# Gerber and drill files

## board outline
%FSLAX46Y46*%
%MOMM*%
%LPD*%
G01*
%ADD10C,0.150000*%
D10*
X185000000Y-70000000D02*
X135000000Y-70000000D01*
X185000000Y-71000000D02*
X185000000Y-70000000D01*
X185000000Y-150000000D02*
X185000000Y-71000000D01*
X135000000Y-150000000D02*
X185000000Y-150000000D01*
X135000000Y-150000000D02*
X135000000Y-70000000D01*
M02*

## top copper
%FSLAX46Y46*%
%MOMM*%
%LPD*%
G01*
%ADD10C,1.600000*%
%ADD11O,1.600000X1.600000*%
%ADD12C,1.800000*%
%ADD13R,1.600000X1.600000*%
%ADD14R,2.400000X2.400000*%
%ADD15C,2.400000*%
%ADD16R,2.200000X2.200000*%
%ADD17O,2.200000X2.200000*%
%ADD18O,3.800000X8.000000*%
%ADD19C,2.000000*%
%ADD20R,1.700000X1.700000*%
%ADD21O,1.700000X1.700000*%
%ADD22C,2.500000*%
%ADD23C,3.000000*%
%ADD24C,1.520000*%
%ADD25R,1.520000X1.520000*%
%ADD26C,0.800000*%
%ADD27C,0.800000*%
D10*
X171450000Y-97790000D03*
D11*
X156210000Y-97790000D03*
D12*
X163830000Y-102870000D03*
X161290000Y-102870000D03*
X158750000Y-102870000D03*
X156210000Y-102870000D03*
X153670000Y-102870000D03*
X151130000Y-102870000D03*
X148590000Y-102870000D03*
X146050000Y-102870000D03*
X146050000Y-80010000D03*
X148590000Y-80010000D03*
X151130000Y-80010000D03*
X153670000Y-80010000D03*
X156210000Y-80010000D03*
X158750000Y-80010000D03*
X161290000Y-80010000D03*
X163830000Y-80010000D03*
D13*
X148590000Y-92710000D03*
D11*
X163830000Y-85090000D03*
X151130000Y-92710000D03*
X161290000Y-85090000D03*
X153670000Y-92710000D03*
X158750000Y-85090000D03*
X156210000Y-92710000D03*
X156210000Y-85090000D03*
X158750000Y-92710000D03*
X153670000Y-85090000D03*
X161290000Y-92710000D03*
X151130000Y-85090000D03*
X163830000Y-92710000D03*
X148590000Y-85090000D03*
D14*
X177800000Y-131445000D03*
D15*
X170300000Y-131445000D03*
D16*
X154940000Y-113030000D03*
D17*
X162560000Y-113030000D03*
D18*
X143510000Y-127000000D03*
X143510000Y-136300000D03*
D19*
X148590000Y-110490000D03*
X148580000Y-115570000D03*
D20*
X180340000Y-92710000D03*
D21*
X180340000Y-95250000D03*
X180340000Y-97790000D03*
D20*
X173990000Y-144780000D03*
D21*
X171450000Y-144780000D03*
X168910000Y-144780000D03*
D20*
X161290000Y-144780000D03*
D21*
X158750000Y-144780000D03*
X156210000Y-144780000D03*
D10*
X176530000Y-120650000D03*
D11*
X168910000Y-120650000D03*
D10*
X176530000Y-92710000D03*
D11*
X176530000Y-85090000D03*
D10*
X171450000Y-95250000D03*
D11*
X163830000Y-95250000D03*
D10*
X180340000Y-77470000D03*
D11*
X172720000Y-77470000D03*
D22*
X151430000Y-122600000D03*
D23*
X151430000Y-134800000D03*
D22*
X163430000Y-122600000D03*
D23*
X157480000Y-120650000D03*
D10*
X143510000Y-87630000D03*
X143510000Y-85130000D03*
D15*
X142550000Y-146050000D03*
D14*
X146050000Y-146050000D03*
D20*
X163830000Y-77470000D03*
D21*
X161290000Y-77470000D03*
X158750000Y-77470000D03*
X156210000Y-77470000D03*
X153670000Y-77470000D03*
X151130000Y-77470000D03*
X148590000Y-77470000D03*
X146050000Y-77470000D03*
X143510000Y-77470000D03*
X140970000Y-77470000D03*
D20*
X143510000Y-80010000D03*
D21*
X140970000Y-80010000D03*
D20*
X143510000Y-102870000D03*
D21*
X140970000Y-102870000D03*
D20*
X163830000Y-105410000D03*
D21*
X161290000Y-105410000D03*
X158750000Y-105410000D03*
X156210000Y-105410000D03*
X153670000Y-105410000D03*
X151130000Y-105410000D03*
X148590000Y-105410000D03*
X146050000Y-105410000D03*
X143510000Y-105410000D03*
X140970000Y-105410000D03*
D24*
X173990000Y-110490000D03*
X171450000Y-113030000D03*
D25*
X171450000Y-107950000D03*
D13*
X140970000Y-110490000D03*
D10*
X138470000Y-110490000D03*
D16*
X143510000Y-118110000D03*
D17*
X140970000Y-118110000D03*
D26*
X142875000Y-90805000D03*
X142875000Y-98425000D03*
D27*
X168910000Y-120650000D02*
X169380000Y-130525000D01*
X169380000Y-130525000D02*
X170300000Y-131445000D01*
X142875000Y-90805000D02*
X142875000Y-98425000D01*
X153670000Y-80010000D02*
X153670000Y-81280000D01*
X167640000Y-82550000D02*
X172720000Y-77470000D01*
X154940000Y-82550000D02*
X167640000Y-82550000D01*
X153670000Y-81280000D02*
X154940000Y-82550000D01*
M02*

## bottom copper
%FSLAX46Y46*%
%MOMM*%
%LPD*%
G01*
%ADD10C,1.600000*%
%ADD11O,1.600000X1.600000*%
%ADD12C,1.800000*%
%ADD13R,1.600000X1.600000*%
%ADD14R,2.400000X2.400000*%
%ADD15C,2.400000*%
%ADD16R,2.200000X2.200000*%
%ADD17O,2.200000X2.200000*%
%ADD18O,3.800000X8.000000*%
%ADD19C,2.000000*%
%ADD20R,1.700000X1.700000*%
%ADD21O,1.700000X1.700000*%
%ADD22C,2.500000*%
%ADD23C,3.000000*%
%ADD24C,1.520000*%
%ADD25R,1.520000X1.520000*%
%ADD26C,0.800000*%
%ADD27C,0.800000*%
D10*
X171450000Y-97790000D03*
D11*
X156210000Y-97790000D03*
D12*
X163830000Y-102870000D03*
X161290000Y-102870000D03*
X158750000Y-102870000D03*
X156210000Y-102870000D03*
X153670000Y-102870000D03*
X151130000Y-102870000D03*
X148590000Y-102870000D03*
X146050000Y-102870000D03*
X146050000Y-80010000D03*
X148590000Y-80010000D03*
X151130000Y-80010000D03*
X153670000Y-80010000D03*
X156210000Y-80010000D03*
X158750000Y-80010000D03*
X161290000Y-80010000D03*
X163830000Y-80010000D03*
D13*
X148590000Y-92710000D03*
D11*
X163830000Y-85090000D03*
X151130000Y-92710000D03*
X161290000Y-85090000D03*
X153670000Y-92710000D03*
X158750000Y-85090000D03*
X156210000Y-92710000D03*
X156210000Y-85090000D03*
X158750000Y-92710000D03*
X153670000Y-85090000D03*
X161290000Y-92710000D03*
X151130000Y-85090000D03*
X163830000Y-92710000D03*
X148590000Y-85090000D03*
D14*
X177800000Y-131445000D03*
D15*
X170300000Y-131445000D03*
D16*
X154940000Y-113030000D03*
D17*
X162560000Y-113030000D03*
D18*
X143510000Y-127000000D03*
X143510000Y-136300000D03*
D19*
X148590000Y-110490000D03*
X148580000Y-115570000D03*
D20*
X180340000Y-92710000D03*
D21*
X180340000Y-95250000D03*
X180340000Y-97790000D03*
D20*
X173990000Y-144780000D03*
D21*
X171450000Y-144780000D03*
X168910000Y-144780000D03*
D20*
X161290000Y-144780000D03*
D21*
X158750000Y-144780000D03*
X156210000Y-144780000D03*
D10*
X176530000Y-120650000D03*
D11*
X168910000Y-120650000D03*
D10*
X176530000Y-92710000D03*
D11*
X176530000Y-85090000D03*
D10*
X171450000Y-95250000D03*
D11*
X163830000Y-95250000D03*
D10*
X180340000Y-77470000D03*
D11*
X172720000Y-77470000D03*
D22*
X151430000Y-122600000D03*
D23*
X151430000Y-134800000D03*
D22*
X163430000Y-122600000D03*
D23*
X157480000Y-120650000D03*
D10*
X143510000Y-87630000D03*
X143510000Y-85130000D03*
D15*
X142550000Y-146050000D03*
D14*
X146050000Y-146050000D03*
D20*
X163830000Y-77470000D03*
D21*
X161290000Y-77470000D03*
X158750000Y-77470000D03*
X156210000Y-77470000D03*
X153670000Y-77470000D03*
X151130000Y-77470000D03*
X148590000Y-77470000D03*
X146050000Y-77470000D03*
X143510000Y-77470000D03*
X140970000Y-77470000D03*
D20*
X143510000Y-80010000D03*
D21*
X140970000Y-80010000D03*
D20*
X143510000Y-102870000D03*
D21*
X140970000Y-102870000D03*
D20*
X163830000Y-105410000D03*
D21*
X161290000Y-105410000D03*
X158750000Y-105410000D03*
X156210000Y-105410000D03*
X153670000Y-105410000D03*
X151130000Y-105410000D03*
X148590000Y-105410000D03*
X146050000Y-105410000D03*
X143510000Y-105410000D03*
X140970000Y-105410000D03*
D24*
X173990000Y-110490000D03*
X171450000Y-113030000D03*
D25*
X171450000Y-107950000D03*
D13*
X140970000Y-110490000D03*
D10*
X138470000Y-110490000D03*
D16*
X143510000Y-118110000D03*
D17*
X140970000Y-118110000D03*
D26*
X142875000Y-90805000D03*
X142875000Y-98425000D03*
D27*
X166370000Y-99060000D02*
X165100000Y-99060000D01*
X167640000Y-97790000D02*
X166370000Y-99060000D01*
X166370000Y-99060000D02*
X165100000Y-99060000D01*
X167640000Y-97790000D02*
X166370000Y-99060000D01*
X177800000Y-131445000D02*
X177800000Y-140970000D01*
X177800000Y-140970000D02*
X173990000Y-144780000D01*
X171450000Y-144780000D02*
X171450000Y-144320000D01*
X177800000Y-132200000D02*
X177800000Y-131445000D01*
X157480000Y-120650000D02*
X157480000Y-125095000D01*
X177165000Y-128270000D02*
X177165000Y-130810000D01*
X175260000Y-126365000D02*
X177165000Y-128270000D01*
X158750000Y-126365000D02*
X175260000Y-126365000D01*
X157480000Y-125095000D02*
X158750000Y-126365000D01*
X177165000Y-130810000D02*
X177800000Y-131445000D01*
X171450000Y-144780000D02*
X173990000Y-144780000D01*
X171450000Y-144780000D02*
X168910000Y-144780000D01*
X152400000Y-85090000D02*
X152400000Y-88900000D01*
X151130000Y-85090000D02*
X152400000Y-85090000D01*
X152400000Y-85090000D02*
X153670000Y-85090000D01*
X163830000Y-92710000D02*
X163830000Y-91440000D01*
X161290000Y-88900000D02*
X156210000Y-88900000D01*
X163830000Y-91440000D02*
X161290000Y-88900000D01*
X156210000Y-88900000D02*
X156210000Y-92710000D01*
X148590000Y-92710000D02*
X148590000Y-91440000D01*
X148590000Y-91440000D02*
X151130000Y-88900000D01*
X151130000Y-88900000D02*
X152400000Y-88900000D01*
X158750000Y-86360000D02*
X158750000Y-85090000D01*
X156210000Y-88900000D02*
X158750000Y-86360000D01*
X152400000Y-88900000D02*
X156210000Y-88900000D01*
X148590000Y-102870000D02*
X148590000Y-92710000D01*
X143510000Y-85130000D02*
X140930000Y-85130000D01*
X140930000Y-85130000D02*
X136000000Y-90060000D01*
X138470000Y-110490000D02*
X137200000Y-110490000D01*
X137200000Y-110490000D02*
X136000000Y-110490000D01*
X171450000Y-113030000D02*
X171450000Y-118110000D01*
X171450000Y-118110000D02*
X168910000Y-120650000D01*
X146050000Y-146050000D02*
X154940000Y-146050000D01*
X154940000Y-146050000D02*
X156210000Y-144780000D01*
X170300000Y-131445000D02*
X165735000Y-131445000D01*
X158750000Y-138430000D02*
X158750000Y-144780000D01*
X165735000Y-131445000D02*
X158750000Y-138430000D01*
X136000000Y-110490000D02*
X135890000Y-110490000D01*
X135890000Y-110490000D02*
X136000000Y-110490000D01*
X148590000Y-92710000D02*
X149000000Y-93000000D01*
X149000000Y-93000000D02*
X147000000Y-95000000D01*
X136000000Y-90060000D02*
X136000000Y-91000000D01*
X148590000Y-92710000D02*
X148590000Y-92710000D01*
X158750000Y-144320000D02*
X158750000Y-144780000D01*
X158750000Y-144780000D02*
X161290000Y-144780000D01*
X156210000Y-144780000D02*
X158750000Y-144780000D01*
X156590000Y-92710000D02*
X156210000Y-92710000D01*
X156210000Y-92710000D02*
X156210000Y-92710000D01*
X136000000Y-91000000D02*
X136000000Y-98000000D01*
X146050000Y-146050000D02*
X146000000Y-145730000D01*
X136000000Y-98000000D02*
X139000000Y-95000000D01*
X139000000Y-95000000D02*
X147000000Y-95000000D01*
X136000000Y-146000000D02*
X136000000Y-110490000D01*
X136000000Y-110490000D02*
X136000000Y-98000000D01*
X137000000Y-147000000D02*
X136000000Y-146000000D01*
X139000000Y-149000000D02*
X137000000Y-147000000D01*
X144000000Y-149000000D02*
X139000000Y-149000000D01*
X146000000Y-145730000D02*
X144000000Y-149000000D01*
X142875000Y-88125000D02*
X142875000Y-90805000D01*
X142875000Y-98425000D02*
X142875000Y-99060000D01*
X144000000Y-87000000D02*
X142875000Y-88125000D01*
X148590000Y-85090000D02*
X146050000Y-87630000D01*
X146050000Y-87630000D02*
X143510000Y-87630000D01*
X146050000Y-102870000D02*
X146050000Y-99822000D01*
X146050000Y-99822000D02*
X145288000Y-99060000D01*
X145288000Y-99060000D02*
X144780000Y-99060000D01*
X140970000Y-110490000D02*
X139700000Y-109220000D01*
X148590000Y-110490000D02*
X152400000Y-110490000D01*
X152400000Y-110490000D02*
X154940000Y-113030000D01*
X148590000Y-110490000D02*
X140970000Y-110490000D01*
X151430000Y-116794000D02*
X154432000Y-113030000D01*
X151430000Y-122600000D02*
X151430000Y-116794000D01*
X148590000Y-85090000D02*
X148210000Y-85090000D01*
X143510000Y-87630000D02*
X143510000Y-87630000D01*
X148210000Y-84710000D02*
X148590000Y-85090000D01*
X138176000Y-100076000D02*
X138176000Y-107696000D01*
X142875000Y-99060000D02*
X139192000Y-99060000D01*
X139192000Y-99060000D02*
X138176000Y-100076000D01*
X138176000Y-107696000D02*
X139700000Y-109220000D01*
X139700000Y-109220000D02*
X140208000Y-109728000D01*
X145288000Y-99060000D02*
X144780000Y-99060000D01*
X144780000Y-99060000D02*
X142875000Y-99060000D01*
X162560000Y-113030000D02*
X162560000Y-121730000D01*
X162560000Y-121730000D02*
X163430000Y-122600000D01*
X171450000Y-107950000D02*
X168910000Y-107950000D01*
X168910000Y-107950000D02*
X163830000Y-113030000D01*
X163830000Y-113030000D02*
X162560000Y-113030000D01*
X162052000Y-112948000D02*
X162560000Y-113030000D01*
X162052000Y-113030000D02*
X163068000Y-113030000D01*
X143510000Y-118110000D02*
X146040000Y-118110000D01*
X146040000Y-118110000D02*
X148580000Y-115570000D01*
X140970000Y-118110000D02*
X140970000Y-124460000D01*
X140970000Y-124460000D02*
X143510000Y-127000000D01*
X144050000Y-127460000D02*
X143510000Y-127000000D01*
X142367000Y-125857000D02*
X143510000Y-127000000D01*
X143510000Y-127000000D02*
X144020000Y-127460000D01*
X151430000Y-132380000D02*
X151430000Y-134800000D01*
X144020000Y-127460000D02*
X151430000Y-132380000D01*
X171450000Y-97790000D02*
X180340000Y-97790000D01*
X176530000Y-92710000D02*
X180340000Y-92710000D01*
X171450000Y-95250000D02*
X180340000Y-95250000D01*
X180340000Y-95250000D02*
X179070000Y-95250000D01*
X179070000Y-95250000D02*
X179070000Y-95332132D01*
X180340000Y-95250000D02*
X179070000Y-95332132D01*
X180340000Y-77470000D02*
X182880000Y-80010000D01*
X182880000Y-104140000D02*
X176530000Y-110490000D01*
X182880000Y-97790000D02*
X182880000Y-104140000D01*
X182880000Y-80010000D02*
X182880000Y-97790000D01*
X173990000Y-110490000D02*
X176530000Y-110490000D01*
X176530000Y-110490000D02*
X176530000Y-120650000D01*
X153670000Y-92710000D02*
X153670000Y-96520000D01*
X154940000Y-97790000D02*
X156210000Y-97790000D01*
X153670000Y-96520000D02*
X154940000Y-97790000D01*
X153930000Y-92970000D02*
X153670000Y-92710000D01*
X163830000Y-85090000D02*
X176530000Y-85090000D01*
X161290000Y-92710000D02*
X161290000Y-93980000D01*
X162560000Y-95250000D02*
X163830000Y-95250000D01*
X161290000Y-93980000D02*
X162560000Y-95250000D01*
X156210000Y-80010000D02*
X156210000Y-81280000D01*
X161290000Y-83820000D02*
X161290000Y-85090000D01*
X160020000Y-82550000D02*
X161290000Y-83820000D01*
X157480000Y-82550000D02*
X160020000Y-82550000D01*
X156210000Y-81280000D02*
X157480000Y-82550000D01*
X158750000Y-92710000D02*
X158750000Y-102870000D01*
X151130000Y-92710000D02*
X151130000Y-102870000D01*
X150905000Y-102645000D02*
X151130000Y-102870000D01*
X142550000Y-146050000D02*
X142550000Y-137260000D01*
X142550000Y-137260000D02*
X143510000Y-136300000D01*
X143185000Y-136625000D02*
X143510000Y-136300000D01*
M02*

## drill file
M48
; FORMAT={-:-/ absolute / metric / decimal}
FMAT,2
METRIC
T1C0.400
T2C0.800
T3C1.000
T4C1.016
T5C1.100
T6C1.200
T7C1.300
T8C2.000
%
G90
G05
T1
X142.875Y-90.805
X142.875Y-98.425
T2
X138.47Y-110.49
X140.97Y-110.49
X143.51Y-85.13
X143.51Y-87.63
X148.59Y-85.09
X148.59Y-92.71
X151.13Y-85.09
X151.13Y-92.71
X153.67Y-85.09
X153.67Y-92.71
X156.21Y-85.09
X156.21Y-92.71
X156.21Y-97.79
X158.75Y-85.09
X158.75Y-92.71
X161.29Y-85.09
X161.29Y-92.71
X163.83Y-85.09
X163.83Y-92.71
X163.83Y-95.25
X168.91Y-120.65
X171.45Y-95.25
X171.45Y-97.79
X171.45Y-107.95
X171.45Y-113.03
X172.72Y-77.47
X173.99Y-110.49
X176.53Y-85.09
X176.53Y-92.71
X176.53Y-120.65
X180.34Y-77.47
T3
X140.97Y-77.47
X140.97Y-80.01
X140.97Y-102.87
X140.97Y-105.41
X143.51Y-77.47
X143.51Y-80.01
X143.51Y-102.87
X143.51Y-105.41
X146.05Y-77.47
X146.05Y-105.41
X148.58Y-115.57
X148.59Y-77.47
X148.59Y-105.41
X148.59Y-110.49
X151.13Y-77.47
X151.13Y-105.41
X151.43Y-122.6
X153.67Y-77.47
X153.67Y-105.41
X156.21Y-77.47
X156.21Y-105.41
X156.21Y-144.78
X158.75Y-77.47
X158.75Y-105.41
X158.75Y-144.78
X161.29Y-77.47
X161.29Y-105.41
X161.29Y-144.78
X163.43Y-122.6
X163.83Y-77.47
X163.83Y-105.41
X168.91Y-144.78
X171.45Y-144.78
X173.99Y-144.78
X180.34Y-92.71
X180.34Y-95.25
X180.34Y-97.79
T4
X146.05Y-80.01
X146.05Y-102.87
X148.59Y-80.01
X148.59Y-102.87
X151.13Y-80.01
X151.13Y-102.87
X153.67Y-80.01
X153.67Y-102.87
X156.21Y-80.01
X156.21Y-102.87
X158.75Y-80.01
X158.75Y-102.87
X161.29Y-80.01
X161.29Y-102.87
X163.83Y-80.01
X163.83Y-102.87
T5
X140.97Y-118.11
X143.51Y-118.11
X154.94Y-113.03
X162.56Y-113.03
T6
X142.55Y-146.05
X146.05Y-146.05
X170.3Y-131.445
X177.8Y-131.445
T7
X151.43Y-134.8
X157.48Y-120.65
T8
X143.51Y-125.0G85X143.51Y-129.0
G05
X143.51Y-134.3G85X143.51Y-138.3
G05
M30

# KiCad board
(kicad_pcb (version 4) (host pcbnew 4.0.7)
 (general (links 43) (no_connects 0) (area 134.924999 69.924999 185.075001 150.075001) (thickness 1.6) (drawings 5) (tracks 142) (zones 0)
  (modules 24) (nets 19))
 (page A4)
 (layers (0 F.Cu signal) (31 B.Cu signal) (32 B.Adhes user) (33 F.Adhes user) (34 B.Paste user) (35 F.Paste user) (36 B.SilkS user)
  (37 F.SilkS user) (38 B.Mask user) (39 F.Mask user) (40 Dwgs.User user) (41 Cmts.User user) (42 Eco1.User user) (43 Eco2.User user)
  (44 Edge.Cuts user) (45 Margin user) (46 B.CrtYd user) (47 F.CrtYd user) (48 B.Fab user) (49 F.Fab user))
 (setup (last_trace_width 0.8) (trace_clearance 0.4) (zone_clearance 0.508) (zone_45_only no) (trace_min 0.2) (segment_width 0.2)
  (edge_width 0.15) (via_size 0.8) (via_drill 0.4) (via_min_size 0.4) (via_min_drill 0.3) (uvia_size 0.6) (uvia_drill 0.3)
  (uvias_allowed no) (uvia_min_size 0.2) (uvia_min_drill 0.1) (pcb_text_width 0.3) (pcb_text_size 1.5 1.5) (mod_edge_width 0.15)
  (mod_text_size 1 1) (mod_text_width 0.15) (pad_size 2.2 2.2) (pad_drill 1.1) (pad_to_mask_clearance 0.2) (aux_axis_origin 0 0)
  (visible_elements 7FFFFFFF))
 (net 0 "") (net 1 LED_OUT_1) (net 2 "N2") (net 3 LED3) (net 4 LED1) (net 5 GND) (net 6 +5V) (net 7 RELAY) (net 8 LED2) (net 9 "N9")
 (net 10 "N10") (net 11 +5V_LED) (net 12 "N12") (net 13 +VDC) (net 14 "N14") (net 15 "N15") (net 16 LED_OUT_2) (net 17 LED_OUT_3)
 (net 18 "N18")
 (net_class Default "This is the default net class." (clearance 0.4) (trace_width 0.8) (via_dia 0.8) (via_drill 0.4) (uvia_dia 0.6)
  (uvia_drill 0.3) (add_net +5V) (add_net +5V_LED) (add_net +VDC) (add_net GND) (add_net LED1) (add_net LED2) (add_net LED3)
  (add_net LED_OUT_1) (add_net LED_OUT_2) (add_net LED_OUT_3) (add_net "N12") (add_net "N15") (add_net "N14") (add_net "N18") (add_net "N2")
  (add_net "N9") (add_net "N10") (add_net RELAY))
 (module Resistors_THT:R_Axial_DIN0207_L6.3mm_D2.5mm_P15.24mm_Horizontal (layer F.Cu) (at 171.45 97.79 180)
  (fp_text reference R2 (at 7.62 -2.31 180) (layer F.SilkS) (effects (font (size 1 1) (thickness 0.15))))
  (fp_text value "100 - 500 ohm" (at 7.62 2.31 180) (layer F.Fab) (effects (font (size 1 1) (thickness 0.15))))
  (pad 1 thru_hole circle (at 0 0 180) (size 1.6 1.6) (drill 0.8) (layers *.Cu *.Mask) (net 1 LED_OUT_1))
  (pad 2 thru_hole oval (at 15.24 0 180) (size 1.6 1.6) (drill 0.8) (layers *.Cu *.Mask) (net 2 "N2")))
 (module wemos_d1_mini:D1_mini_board (layer B.Cu) (at 153.67 91.44 90)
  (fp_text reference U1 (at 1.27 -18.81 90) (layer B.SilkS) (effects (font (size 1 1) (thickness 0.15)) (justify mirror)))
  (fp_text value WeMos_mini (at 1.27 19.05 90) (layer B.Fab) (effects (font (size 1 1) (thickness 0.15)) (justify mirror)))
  (pad 8 thru_hole circle (at -11.43 10.16 90) (size 1.8 1.8) (drill 1.016) (layers *.Cu *.Mask B.SilkS))
  (pad 7 thru_hole circle (at -11.43 7.62 90) (size 1.8 1.8) (drill 1.016) (layers *.Cu *.Mask B.SilkS))
  (pad 6 thru_hole circle (at -11.43 5.08 90) (size 1.8 1.8) (drill 1.016) (layers *.Cu *.Mask B.SilkS) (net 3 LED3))
  (pad 5 thru_hole circle (at -11.43 2.54 90) (size 1.8 1.8) (drill 1.016) (layers *.Cu *.Mask B.SilkS))
  (pad 4 thru_hole circle (at -11.43 0 90) (size 1.8 1.8) (drill 1.016) (layers *.Cu *.Mask B.SilkS))
  (pad 3 thru_hole circle (at -11.43 -2.54 90) (size 1.8 1.8) (drill 1.016) (layers *.Cu *.Mask B.SilkS) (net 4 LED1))
  (pad 2 thru_hole circle (at -11.43 -5.08 90) (size 1.8 1.8) (drill 1.016) (layers *.Cu *.Mask B.SilkS) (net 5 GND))
  (pad 1 thru_hole circle (at -11.43 -7.62 90) (size 1.8 1.8) (drill 1.016) (layers *.Cu *.Mask B.SilkS) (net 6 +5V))
  (pad 16 thru_hole circle (at 11.43 -7.62 90) (size 1.8 1.8) (drill 1.016) (layers *.Cu *.Mask B.SilkS))
  (pad 15 thru_hole circle (at 11.43 -5.08 90) (size 1.8 1.8) (drill 1.016) (layers *.Cu *.Mask B.SilkS))
  (pad 14 thru_hole circle (at 11.43 -2.54 90) (size 1.8 1.8) (drill 1.016) (layers *.Cu *.Mask B.SilkS))
  (pad 13 thru_hole circle (at 11.43 0 90) (size 1.8 1.8) (drill 1.016) (layers *.Cu *.Mask B.SilkS) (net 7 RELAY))
  (pad 12 thru_hole circle (at 11.43 2.54 90) (size 1.8 1.8) (drill 1.016) (layers *.Cu *.Mask B.SilkS) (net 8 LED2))
  (pad 11 thru_hole circle (at 11.43 5.08 90) (size 1.8 1.8) (drill 1.016) (layers *.Cu *.Mask B.SilkS))
  (pad 10 thru_hole circle (at 11.43 7.62 90) (size 1.8 1.8) (drill 1.016) (layers *.Cu *.Mask B.SilkS))
  (pad 9 thru_hole circle (at 11.43 10.16 90) (size 1.8 1.8) (drill 1.016) (layers *.Cu *.Mask B.SilkS)))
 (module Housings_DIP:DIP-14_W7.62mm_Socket (layer F.Cu) (at 148.59 92.71 90)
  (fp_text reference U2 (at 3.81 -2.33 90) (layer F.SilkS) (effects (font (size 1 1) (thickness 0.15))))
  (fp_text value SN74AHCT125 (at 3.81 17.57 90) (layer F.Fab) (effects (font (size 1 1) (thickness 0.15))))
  (pad 1 thru_hole rect (at 0 0 90) (size 1.6 1.6) (drill 0.8) (layers *.Cu *.Mask) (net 5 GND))
  (pad 8 thru_hole oval (at 7.62 15.24 90) (size 1.6 1.6) (drill 0.8) (layers *.Cu *.Mask) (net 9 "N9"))
  (pad 2 thru_hole oval (at 0 2.54 90) (size 1.6 1.6) (drill 0.8) (layers *.Cu *.Mask) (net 4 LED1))
  (pad 9 thru_hole oval (at 7.62 12.7 90) (size 1.6 1.6) (drill 0.8) (layers *.Cu *.Mask) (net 8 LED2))
  (pad 3 thru_hole oval (at 0 5.08 90) (size 1.6 1.6) (drill 0.8) (layers *.Cu *.Mask) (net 2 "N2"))
  (pad 10 thru_hole oval (at 7.62 10.16 90) (size 1.6 1.6) (drill 0.8) (layers *.Cu *.Mask) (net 5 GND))
  (pad 4 thru_hole oval (at 0 7.62 90) (size 1.6 1.6) (drill 0.8) (layers *.Cu *.Mask) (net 5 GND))
  (pad 11 thru_hole oval (at 7.62 7.62 90) (size 1.6 1.6) (drill 0.8) (layers *.Cu *.Mask))
  (pad 5 thru_hole oval (at 0 10.16 90) (size 1.6 1.6) (drill 0.8) (layers *.Cu *.Mask) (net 3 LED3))
  (pad 12 thru_hole oval (at 7.62 5.08 90) (size 1.6 1.6) (drill 0.8) (layers *.Cu *.Mask) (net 5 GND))
  (pad 6 thru_hole oval (at 0 12.7 90) (size 1.6 1.6) (drill 0.8) (layers *.Cu *.Mask) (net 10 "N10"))
  (pad 13 thru_hole oval (at 7.62 2.54 90) (size 1.6 1.6) (drill 0.8) (layers *.Cu *.Mask) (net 5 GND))
  (pad 7 thru_hole oval (at 0 15.24 90) (size 1.6 1.6) (drill 0.8) (layers *.Cu *.Mask) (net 5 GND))
  (pad 14 thru_hole oval (at 7.62 0 90) (size 1.6 1.6) (drill 0.8) (layers *.Cu *.Mask) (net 6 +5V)))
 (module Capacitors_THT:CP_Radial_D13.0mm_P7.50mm (layer F.Cu) (at 177.8 131.445 180)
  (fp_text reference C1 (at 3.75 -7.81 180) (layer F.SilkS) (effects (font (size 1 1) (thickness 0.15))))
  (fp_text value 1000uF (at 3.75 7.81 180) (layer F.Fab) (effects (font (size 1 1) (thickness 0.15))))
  (pad 1 thru_hole rect (at 0 0 180) (size 2.4 2.4) (drill 1.2) (layers *.Cu *.Mask) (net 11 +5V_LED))
  (pad 2 thru_hole circle (at 7.5 0 180) (size 2.4 2.4) (drill 1.2) (layers *.Cu *.Mask) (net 5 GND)))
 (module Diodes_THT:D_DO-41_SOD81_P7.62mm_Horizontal (layer F.Cu) (at 154.94 113.03)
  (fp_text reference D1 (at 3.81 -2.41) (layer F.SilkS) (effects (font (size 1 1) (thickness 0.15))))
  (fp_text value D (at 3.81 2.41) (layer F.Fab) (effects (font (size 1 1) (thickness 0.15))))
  (pad 1 thru_hole rect (at 0 0) (size 2.2 2.2) (drill 1.1) (layers *.Cu *.Mask) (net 6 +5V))
  (pad 2 thru_hole oval (at 7.62 0) (size 2.2 2.2) (drill 1.1) (layers *.Cu *.Mask) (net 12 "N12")))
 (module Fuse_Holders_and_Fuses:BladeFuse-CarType (layer F.Cu) (at 143.51 127 270)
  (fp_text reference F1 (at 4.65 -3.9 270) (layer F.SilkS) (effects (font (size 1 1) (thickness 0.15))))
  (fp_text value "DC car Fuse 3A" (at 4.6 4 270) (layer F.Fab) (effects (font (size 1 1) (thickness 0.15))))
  (pad 1 thru_hole oval (at 0 0 270) (size 8 3.8) (drill oval 6 2) (layers *.Cu *.Mask) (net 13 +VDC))
  (pad 2 thru_hole oval (at 9.3 0 270) (size 8 3.8) (drill oval 6 2) (layers *.Cu *.Mask) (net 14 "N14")))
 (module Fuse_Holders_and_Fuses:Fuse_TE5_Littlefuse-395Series (layer F.Cu) (at 148.59 110.49 270)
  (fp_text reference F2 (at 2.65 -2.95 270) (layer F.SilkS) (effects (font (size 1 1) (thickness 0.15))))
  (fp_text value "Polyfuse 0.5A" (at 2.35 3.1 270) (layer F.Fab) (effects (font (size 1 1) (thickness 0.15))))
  (pad 1 thru_hole circle (at 0 0 270) (size 2 2) (drill 1) (layers *.Cu *.Mask) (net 6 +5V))
  (pad 2 thru_hole circle (at 5.08 0.01 270) (size 2 2) (drill 1) (layers *.Cu *.Mask) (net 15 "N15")))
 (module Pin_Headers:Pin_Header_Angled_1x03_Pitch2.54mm (layer F.Cu) (at 180.34 92.71)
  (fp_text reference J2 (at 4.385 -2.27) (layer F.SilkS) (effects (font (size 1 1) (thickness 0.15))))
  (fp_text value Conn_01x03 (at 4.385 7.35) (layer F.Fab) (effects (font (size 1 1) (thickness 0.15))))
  (pad 1 thru_hole rect (at 0 0) (size 1.7 1.7) (drill 1) (layers *.Cu *.Mask) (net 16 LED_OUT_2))
  (pad 2 thru_hole oval (at 0 2.54) (size 1.7 1.7) (drill 1) (layers *.Cu *.Mask) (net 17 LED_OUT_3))
  (pad 3 thru_hole oval (at 0 5.08) (size 1.7 1.7) (drill 1) (layers *.Cu *.Mask) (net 1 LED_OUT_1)))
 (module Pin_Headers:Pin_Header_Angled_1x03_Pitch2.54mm (layer F.Cu) (at 173.99 144.78 270)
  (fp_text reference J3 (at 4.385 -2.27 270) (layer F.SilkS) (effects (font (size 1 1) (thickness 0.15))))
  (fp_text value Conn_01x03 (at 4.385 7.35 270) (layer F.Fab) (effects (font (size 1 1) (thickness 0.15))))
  (pad 1 thru_hole rect (at 0 0 270) (size 1.7 1.7) (drill 1) (layers *.Cu *.Mask) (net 11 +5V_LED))
  (pad 2 thru_hole oval (at 0 2.54 270) (size 1.7 1.7) (drill 1) (layers *.Cu *.Mask) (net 11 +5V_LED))
  (pad 3 thru_hole oval (at 0 5.08 270) (size 1.7 1.7) (drill 1) (layers *.Cu *.Mask) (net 11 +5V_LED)))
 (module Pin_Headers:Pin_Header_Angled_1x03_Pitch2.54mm (layer F.Cu) (at 161.29 144.78 270)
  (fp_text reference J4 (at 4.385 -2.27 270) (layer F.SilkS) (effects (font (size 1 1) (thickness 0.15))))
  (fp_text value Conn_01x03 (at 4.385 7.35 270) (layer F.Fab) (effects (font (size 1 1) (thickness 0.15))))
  (pad 1 thru_hole rect (at 0 0 270) (size 1.7 1.7) (drill 1) (layers *.Cu *.Mask) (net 5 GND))
  (pad 2 thru_hole oval (at 0 2.54 270) (size 1.7 1.7) (drill 1) (layers *.Cu *.Mask) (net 5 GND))
  (pad 3 thru_hole oval (at 0 5.08 270) (size 1.7 1.7) (drill 1) (layers *.Cu *.Mask) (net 5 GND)))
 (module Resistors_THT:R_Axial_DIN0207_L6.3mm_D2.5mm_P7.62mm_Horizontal (layer F.Cu) (at 176.53 120.65 180)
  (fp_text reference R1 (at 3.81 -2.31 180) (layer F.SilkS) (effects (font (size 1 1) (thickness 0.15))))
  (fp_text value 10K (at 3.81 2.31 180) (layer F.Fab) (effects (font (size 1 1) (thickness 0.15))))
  (pad 1 thru_hole circle (at 0 0 180) (size 1.6 1.6) (drill 0.8) (layers *.Cu *.Mask) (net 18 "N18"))
  (pad 2 thru_hole oval (at 7.62 0 180) (size 1.6 1.6) (drill 0.8) (layers *.Cu *.Mask) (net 5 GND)))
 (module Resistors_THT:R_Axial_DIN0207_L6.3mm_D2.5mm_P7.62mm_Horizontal (layer F.Cu) (at 176.53 92.71 90)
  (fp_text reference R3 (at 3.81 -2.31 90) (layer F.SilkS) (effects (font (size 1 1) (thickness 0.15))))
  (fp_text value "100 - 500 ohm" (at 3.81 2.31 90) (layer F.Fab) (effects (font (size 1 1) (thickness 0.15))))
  (pad 1 thru_hole circle (at 0 0 90) (size 1.6 1.6) (drill 0.8) (layers *.Cu *.Mask) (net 16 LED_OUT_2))
  (pad 2 thru_hole oval (at 7.62 0 90) (size 1.6 1.6) (drill 0.8) (layers *.Cu *.Mask) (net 9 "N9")))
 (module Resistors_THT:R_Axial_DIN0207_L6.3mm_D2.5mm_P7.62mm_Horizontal (layer F.Cu) (at 171.45 95.25 180)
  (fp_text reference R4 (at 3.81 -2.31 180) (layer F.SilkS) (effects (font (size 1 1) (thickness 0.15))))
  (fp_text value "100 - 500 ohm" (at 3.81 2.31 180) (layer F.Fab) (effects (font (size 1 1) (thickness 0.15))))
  (pad 1 thru_hole circle (at 0 0 180) (size 1.6 1.6) (drill 0.8) (layers *.Cu *.Mask) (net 17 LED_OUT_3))
  (pad 2 thru_hole oval (at 7.62 0 180) (size 1.6 1.6) (drill 0.8) (layers *.Cu *.Mask) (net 10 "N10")))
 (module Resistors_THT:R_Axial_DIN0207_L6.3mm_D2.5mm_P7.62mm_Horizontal (layer F.Cu) (at 180.34 77.47 180)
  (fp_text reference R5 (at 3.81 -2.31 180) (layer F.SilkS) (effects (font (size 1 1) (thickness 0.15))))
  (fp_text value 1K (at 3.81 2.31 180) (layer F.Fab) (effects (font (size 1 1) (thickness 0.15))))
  (pad 1 thru_hole circle (at 0 0 180) (size 1.6 1.6) (drill 0.8) (layers *.Cu *.Mask) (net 18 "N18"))
  (pad 2 thru_hole oval (at 7.62 0 180) (size 1.6 1.6) (drill 0.8) (layers *.Cu *.Mask) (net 7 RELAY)))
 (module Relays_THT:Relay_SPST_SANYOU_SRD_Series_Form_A (layer F.Cu) (at 157.48 120.65 270)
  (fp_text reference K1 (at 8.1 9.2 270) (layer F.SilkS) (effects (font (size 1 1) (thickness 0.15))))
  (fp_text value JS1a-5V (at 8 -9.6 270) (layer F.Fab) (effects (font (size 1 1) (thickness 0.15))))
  (pad 5 thru_hole circle (at 1.95 6.05) (size 2.5 2.5) (drill 1) (layers *.Cu *.Mask) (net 6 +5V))
  (pad 4 thru_hole circle (at 14.15 6.05) (size 3 3) (drill 1.3) (layers *.Cu *.Mask) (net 13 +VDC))
  (pad 2 thru_hole circle (at 1.95 -5.95) (size 2.5 2.5) (drill 1) (layers *.Cu *.Mask) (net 12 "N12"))
  (pad 1 thru_hole circle (at 0 0) (size 3 3) (drill 1.3) (layers *.Cu *.Mask) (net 11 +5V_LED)))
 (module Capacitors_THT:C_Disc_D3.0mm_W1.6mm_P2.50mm (layer F.Cu) (at 143.51 87.63 90)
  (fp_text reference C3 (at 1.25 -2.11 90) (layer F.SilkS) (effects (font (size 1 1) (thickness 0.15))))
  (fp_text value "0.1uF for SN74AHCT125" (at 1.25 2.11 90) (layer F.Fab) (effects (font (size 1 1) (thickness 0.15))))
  (pad 1 thru_hole circle (at 0 0 90) (size 1.6 1.6) (drill 0.8) (layers *.Cu *.Mask) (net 6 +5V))
  (pad 2 thru_hole circle (at 2.5 0 90) (size 1.6 1.6) (drill 0.8) (layers *.Cu *.Mask) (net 5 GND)))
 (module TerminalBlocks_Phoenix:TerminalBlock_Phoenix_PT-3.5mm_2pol (layer F.Cu) (at 146.05 146.05 180)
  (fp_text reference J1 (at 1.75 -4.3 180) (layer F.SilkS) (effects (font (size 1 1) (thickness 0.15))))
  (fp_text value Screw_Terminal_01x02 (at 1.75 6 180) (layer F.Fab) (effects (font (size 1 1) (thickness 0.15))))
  (pad 2 thru_hole circle (at 3.5 0 180) (size 2.4 2.4) (drill 1.2) (layers *.Cu *.Mask) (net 14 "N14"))
  (pad 1 thru_hole rect (at 0 0 180) (size 2.4 2.4) (drill 1.2) (layers *.Cu *.Mask) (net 5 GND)))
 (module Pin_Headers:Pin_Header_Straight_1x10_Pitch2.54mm (layer F.Cu) (at 163.83 77.47 270)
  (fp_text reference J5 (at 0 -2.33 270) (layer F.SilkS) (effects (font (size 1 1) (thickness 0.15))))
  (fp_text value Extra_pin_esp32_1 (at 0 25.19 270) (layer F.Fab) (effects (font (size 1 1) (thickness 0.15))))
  (pad 1 thru_hole rect (at 0 0 270) (size 1.7 1.7) (drill 1) (layers *.Cu *.Mask))
  (pad 2 thru_hole oval (at 0 2.54 270) (size 1.7 1.7) (drill 1) (layers *.Cu *.Mask))
  (pad 3 thru_hole oval (at 0 5.08 270) (size 1.7 1.7) (drill 1) (layers *.Cu *.Mask))
  (pad 4 thru_hole oval (at 0 7.62 270) (size 1.7 1.7) (drill 1) (layers *.Cu *.Mask))
  (pad 5 thru_hole oval (at 0 10.16 270) (size 1.7 1.7) (drill 1) (layers *.Cu *.Mask))
  (pad 6 thru_hole oval (at 0 12.7 270) (size 1.7 1.7) (drill 1) (layers *.Cu *.Mask))
  (pad 7 thru_hole oval (at 0 15.24 270) (size 1.7 1.7) (drill 1) (layers *.Cu *.Mask))
  (pad 8 thru_hole oval (at 0 17.78 270) (size 1.7 1.7) (drill 1) (layers *.Cu *.Mask))
  (pad 9 thru_hole oval (at 0 20.32 270) (size 1.7 1.7) (drill 1) (layers *.Cu *.Mask))
  (pad 10 thru_hole oval (at 0 22.86 270) (size 1.7 1.7) (drill 1) (layers *.Cu *.Mask)))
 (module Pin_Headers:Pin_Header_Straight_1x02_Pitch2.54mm (layer F.Cu) (at 143.51 80.01 270)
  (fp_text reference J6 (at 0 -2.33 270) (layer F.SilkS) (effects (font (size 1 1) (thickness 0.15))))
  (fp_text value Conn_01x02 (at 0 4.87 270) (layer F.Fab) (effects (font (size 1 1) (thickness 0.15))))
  (pad 1 thru_hole rect (at 0 0 270) (size 1.7 1.7) (drill 1) (layers *.Cu *.Mask))
  (pad 2 thru_hole oval (at 0 2.54 270) (size 1.7 1.7) (drill 1) (layers *.Cu *.Mask)))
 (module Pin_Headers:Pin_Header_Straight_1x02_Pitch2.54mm (layer F.Cu) (at 143.51 102.87 270)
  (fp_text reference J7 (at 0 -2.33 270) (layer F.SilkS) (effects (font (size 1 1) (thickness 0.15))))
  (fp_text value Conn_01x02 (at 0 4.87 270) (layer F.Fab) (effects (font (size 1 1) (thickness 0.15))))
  (pad 1 thru_hole rect (at 0 0 270) (size 1.7 1.7) (drill 1) (layers *.Cu *.Mask))
  (pad 2 thru_hole oval (at 0 2.54 270) (size 1.7 1.7) (drill 1) (layers *.Cu *.Mask)))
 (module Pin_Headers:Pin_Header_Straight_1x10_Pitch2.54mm (layer F.Cu) (at 163.83 105.41 270)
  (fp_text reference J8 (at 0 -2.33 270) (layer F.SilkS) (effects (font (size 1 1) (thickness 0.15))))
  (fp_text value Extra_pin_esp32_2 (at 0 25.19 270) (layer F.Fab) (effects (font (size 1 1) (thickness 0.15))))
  (pad 1 thru_hole rect (at 0 0 270) (size 1.7 1.7) (drill 1) (layers *.Cu *.Mask))
  (pad 2 thru_hole oval (at 0 2.54 270) (size 1.7 1.7) (drill 1) (layers *.Cu *.Mask))
  (pad 3 thru_hole oval (at 0 5.08 270) (size 1.7 1.7) (drill 1) (layers *.Cu *.Mask))
  (pad 4 thru_hole oval (at 0 7.62 270) (size 1.7 1.7) (drill 1) (layers *.Cu *.Mask))
  (pad 5 thru_hole oval (at 0 10.16 270) (size 1.7 1.7) (drill 1) (layers *.Cu *.Mask))
  (pad 6 thru_hole oval (at 0 12.7 270) (size 1.7 1.7) (drill 1) (layers *.Cu *.Mask))
  (pad 7 thru_hole oval (at 0 15.24 270) (size 1.7 1.7) (drill 1) (layers *.Cu *.Mask))
  (pad 8 thru_hole oval (at 0 17.78 270) (size 1.7 1.7) (drill 1) (layers *.Cu *.Mask))
  (pad 9 thru_hole oval (at 0 20.32 270) (size 1.7 1.7) (drill 1) (layers *.Cu *.Mask))
  (pad 10 thru_hole oval (at 0 22.86 270) (size 1.7 1.7) (drill 1) (layers *.Cu *.Mask)))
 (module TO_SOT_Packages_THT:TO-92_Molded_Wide (layer F.Cu) (at 171.45 107.95 270)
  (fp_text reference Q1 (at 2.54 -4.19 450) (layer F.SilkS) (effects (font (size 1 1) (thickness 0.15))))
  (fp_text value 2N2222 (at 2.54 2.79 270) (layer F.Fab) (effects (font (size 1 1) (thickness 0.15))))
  (pad 2 thru_hole circle (at 2.54 -2.54) (size 1.52 1.52) (drill 0.8) (layers *.Cu *.Mask) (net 18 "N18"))
  (pad 3 thru_hole circle (at 5.08 0) (size 1.52 1.52) (drill 0.8) (layers *.Cu *.Mask) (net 5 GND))
  (pad 1 thru_hole rect (at 0 0) (size 1.52 1.52) (drill 0.8) (layers *.Cu *.Mask) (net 12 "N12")))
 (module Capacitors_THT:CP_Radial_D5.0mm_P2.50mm (layer F.Cu) (at 140.97 110.49 180)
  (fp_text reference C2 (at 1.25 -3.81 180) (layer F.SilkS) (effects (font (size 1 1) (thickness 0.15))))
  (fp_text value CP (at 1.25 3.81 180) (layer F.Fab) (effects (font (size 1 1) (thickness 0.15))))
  (pad 1 thru_hole rect (at 0 0 180) (size 1.6 1.6) (drill 0.8) (layers *.Cu *.Mask) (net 6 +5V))
  (pad 2 thru_hole circle (at 2.5 0 180) (size 1.6 1.6) (drill 0.8) (layers *.Cu *.Mask) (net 5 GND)))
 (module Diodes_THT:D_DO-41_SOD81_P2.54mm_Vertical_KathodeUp (layer F.Cu) (at 143.51 118.11 180)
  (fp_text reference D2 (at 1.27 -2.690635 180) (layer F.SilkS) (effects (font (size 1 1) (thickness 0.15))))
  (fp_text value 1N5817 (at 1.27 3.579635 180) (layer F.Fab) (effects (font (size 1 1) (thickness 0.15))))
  (pad 1 thru_hole rect (at 0 0 180) (size 2.2 2.2) (drill 1.1) (layers *.Cu *.Mask) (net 15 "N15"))
  (pad 2 thru_hole oval (at 2.54 0 180) (size 2.2 2.2) (drill 1.1) (layers *.Cu *.Mask) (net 13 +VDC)))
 (gr_line (start 185 70) (end 135 70) (angle 90) (layer Edge.Cuts) (width 0.15))
 (gr_line (start 185 71) (end 185 70) (angle 90) (layer Edge.Cuts) (width 0.15))
 (gr_line (start 185 150) (end 185 71) (angle 90) (layer Edge.Cuts) (width 0.15))
 (gr_line (start 135 150) (end 185 150) (angle 90) (layer Edge.Cuts) (width 0.15))
 (gr_line (start 135 150) (end 135 70) (angle 90) (layer Edge.Cuts) (width 0.15))
 (segment (start 166.37 99.06) (end 165.1 99.06) (width 0.8) (layer B.Cu) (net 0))
 (segment (start 167.64 97.79) (end 166.37 99.06) (width 0.8) (layer B.Cu) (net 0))
 (segment (start 166.37 99.06) (end 165.1 99.06) (width 0.8) (layer B.Cu) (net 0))
 (segment (start 167.64 97.79) (end 166.37 99.06) (width 0.8) (layer B.Cu) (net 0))
 (segment (start 177.8 131.445) (end 177.8 140.97) (width 0.8) (layer B.Cu) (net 11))
 (segment (start 177.8 140.97) (end 173.99 144.78) (width 0.8) (layer B.Cu) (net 11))
 (segment (start 171.45 144.78) (end 171.45 144.32) (width 0.8) (layer B.Cu) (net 11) (status 30))
 (segment (start 177.8 132.2) (end 177.8 131.445) (width 0.8) (layer B.Cu) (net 11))
 (segment (start 157.48 120.65) (end 157.48 125.095) (width 0.8) (layer B.Cu) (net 11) (status 10))
 (segment (start 177.165 128.27) (end 177.165 130.81) (width 0.8) (layer B.Cu) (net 11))
 (segment (start 175.26 126.365) (end 177.165 128.27) (width 0.8) (layer B.Cu) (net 11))
 (segment (start 158.75 126.365) (end 175.26 126.365) (width 0.8) (layer B.Cu) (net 11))
 (segment (start 157.48 125.095) (end 158.75 126.365) (width 0.8) (layer B.Cu) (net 11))
 (segment (start 177.165 130.81) (end 177.8 131.445) (width 0.8) (layer B.Cu) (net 11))
 (segment (start 171.45 144.78) (end 173.99 144.78) (width 0.8) (layer B.Cu) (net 11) (status 30))
 (segment (start 171.45 144.78) (end 168.91 144.78) (width 0.8) (layer B.Cu) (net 11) (status 30))
 (segment (start 152.4 85.09) (end 152.4 88.9) (width 0.8) (layer B.Cu) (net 5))
 (segment (start 151.13 85.09) (end 152.4 85.09) (width 0.8) (layer B.Cu) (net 5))
 (segment (start 152.4 85.09) (end 153.67 85.09) (width 0.8) (layer B.Cu) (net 5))
 (segment (start 163.83 92.71) (end 163.83 91.44) (width 0.8) (layer B.Cu) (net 5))
 (segment (start 161.29 88.9) (end 156.21 88.9) (width 0.8) (layer B.Cu) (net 5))
 (segment (start 163.83 91.44) (end 161.29 88.9) (width 0.8) (layer B.Cu) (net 5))
 (segment (start 156.21 88.9) (end 156.21 92.71) (width 0.8) (layer B.Cu) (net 5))
 (segment (start 148.59 92.71) (end 148.59 91.44) (width 0.8) (layer B.Cu) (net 5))
 (segment (start 148.59 91.44) (end 151.13 88.9) (width 0.8) (layer B.Cu) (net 5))
 (segment (start 151.13 88.9) (end 152.4 88.9) (width 0.8) (layer B.Cu) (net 5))
 (segment (start 158.75 86.36) (end 158.75 85.09) (width 0.8) (layer B.Cu) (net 5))
 (segment (start 156.21 88.9) (end 158.75 86.36) (width 0.8) (layer B.Cu) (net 5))
 (segment (start 152.4 88.9) (end 156.21 88.9) (width 0.8) (layer B.Cu) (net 5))
 (segment (start 148.59 102.87) (end 148.59 92.71) (width 0.8) (layer B.Cu) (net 5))
 (segment (start 143.51 85.13) (end 140.93 85.13) (width 0.8) (layer B.Cu) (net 5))
 (segment (start 140.93 85.13) (end 136 90.06) (width 0.8) (layer B.Cu) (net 5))
 (segment (start 138.47 110.49) (end 137.2 110.49) (width 0.8) (layer B.Cu) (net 5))
 (segment (start 137.2 110.49) (end 136 110.49) (width 0.8) (layer B.Cu) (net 5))
 (segment (start 171.45 113.03) (end 171.45 118.11) (width 0.8) (layer B.Cu) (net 5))
 (segment (start 171.45 118.11) (end 168.91 120.65) (width 0.8) (layer B.Cu) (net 5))
 (segment (start 146.05 146.05) (end 154.94 146.05) (width 0.8) (layer B.Cu) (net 5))
 (segment (start 154.94 146.05) (end 156.21 144.78) (width 0.8) (layer B.Cu) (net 5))
 (segment (start 170.3 131.445) (end 165.735 131.445) (width 0.8) (layer B.Cu) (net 5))
 (segment (start 158.75 138.43) (end 158.75 144.78) (width 0.8) (layer B.Cu) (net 5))
 (segment (start 165.735 131.445) (end 158.75 138.43) (width 0.8) (layer B.Cu) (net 5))
 (segment (start 136 110.49) (end 135.89 110.49) (width 0.8) (layer B.Cu) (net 5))
 (segment (start 135.89 110.49) (end 136 110.49) (width 0.8) (layer B.Cu) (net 5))
 (segment (start 168.91 120.65) (end 169.38 130.525) (width 0.8) (layer F.Cu) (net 5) (status 10))
 (segment (start 169.38 130.525) (end 170.3 131.445) (width 0.8) (layer F.Cu) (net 5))
 (segment (start 148.59 92.71) (end 149 93) (width 0.8) (layer B.Cu) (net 5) (status 10))
 (segment (start 149 93) (end 147 95) (width 0.8) (layer B.Cu) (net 5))
 (segment (start 136 90.06) (end 136 91) (width 0.8) (layer B.Cu) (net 5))
 (segment (start 148.59 92.71) (end 148.59 92.71) (width 0.8) (layer B.Cu) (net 5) (status 10))
 (segment (start 158.75 144.32) (end 158.75 144.78) (width 0.8) (layer B.Cu) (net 5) (status 30))
 (segment (start 158.75 144.78) (end 161.29 144.78) (width 0.8) (layer B.Cu) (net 5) (status 30))
 (segment (start 156.21 144.78) (end 158.75 144.78) (width 0.8) (layer B.Cu) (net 5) (status 30))
 (segment (start 156.59 92.71) (end 156.21 92.71) (width 0.8) (layer B.Cu) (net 5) (status 30))
 (segment (start 156.21 92.71) (end 156.21 92.71) (width 0.8) (layer B.Cu) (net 5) (status 30))
 (segment (start 136 91) (end 136 98) (width 0.8) (layer B.Cu) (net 5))
 (segment (start 146.05 146.05) (end 146 145.73) (width 0.8) (layer B.Cu) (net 5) (status 30))
 (segment (start 136 98) (end 139 95) (width 0.8) (layer B.Cu) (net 5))
 (segment (start 139 95) (end 147 95) (width 0.8) (layer B.Cu) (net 5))
 (segment (start 136 146) (end 136 110.49) (width 0.8) (layer B.Cu) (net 5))
 (segment (start 136 110.49) (end 136 98) (width 0.8) (layer B.Cu) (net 5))
 (segment (start 137 147) (end 136 146) (width 0.8) (layer B.Cu) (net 5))
 (segment (start 139 149) (end 137 147) (width 0.8) (layer B.Cu) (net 5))
 (segment (start 144 149) (end 139 149) (width 0.8) (layer B.Cu) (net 5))
 (segment (start 146 145.73) (end 144 149) (width 0.8) (layer B.Cu) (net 5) (status 10))
 (segment (start 142.875 88.125) (end 142.875 90.805) (width 0.8) (layer B.Cu) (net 6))
 (segment (start 142.875 90.805) (end 142.875 98.425) (width 0.8) (layer F.Cu) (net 6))
 (via (at 142.875 90.805) (size 0.8) (drill 0.4) (layers F.Cu B.Cu) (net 6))
 (segment (start 142.875 98.425) (end 142.875 99.06) (width 0.8) (layer B.Cu) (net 6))
 (via (at 142.875 98.425) (size 0.8) (drill 0.4) (layers F.Cu B.Cu) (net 6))
 (segment (start 144 87) (end 142.875 88.125) (width 0.8) (layer B.Cu) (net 6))
 (segment (start 148.59 85.09) (end 146.05 87.63) (width 0.8) (layer B.Cu) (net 6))
 (segment (start 146.05 87.63) (end 143.51 87.63) (width 0.8) (layer B.Cu) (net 6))
 (segment (start 146.05 102.87) (end 146.05 99.822) (width 0.8) (layer B.Cu) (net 6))
 (segment (start 146.05 99.822) (end 145.288 99.06) (width 0.8) (layer B.Cu) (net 6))
 (segment (start 145.288 99.06) (end 144.78 99.06) (width 0.8) (layer B.Cu) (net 6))
 (segment (start 140.97 110.49) (end 139.7 109.22) (width 0.8) (layer B.Cu) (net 6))
 (segment (start 148.59 110.49) (end 152.4 110.49) (width 0.8) (layer B.Cu) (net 6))
 (segment (start 152.4 110.49) (end 154.94 113.03) (width 0.8) (layer B.Cu) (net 6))
 (segment (start 148.59 110.49) (end 140.97 110.49) (width 0.8) (layer B.Cu) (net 6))
 (segment (start 151.43 116.794) (end 154.432 113.03) (width 0.8) (layer B.Cu) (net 6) (status 20))
 (segment (start 151.43 122.6) (end 151.43 116.794) (width 0.8) (layer B.Cu) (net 6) (status 10))
 (segment (start 148.59 85.09) (end 148.21 85.09) (width 0.8) (layer B.Cu) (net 6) (status 30))
 (segment (start 143.51 87.63) (end 143.51 87.63) (width 0.8) (layer B.Cu) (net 6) (status 30))
 (segment (start 148.21 84.71) (end 148.59 85.09) (width 0.8) (layer B.Cu) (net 6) (status 30))
 (segment (start 138.176 100.076) (end 138.176 107.696) (width 0.8) (layer B.Cu) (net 6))
 (segment (start 142.875 99.06) (end 139.192 99.06) (width 0.8) (layer B.Cu) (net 6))
 (segment (start 139.192 99.06) (end 138.176 100.076) (width 0.8) (layer B.Cu) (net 6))
 (segment (start 138.176 107.696) (end 139.7 109.22) (width 0.8) (layer B.Cu) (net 6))
 (segment (start 139.7 109.22) (end 140.208 109.728) (width 0.8) (layer B.Cu) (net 6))
 (segment (start 145.288 99.06) (end 144.78 99.06) (width 0.8) (layer B.Cu) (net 6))
 (segment (start 144.78 99.06) (end 142.875 99.06) (width 0.8) (layer B.Cu) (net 6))
 (segment (start 162.56 113.03) (end 162.56 121.73) (width 0.8) (layer B.Cu) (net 12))
 (segment (start 162.56 121.73) (end 163.43 122.6) (width 0.8) (layer B.Cu) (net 12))
 (segment (start 171.45 107.95) (end 168.91 107.95) (width 0.8) (layer B.Cu) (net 12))
 (segment (start 168.91 107.95) (end 163.83 113.03) (width 0.8) (layer B.Cu) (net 12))
 (segment (start 163.83 113.03) (end 162.56 113.03) (width 0.8) (layer B.Cu) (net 12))
 (segment (start 162.052 112.948) (end 162.56 113.03) (width 0.8) (layer B.Cu) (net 12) (status 30))
 (segment (start 162.052 113.03) (end 163.068 113.03) (width 0.8) (layer B.Cu) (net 12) (status 30))
 (segment (start 143.51 118.11) (end 146.04 118.11) (width 0.8) (layer B.Cu) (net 15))
 (segment (start 146.04 118.11) (end 148.58 115.57) (width 0.8) (layer B.Cu) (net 15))
 (segment (start 140.97 118.11) (end 140.97 124.46) (width 0.8) (layer B.Cu) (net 13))
 (segment (start 140.97 124.46) (end 143.51 127) (width 0.8) (layer B.Cu) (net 13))
 (segment (start 144.05 127.46) (end 143.51 127) (width 0.8) (layer B.Cu) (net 13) (status 30))
 (segment (start 142.367 125.857) (end 143.51 127) (width 0.8) (layer B.Cu) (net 13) (status 30))
 (segment (start 143.51 127) (end 144.02 127.46) (width 0.8) (layer B.Cu) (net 13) (status 30))
 (segment (start 151.43 132.38) (end 151.43 134.8) (width 0.8) (layer B.Cu) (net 13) (status 20))
 (segment (start 144.02 127.46) (end 151.43 132.38) (width 0.8) (layer B.Cu) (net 13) (status 10))
 (segment (start 171.45 97.79) (end 180.34 97.79) (width 0.8) (layer B.Cu) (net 1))
 (segment (start 176.53 92.71) (end 180.34 92.71) (width 0.8) (layer B.Cu) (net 16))
 (segment (start 171.45 95.25) (end 180.34 95.25) (width 0.8) (layer B.Cu) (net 17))
 (segment (start 180.34 95.25) (end 179.07 95.25) (width 0.8) (layer B.Cu) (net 17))
 (segment (start 179.07 95.25) (end 179.07 95.332132) (width 0.8) (layer B.Cu) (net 17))
 (segment (start 180.34 95.25) (end 179.07 95.332132) (width 0.8) (layer B.Cu) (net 17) (status 20))
 (segment (start 180.34 77.47) (end 182.88 80.01) (width 0.8) (layer B.Cu) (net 18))
 (segment (start 182.88 104.14) (end 176.53 110.49) (width 0.8) (layer B.Cu) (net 18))
 (segment (start 182.88 97.79) (end 182.88 104.14) (width 0.8) (layer B.Cu) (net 18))
 (segment (start 182.88 80.01) (end 182.88 97.79) (width 0.8) (layer B.Cu) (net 18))
 (segment (start 173.99 110.49) (end 176.53 110.49) (width 0.8) (layer B.Cu) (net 18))
 (segment (start 176.53 110.49) (end 176.53 120.65) (width 0.8) (layer B.Cu) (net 18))
 (segment (start 153.67 92.71) (end 153.67 96.52) (width 0.8) (layer B.Cu) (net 2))
 (segment (start 154.94 97.79) (end 156.21 97.79) (width 0.8) (layer B.Cu) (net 2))
 (segment (start 153.67 96.52) (end 154.94 97.79) (width 0.8) (layer B.Cu) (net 2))
 (segment (start 153.93 92.97) (end 153.67 92.71) (width 0.8) (layer B.Cu) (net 2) (status 30))
 (segment (start 163.83 85.09) (end 176.53 85.09) (width 0.8) (layer B.Cu) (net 9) (status 20))
 (segment (start 161.29 92.71) (end 161.29 93.98) (width 0.8) (layer B.Cu) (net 10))
 (segment (start 162.56 95.25) (end 163.83 95.25) (width 0.8) (layer B.Cu) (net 10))
 (segment (start 161.29 93.98) (end 162.56 95.25) (width 0.8) (layer B.Cu) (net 10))
 (segment (start 153.67 80.01) (end 153.67 81.28) (width 0.8) (layer F.Cu) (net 7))
 (segment (start 167.64 82.55) (end 172.72 77.47) (width 0.8) (layer F.Cu) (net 7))
 (segment (start 154.94 82.55) (end 167.64 82.55) (width 0.8) (layer F.Cu) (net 7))
 (segment (start 153.67 81.28) (end 154.94 82.55) (width 0.8) (layer F.Cu) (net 7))
 (segment (start 156.21 80.01) (end 156.21 81.28) (width 0.8) (layer B.Cu) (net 8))
 (segment (start 161.29 83.82) (end 161.29 85.09) (width 0.8) (layer B.Cu) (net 8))
 (segment (start 160.02 82.55) (end 161.29 83.82) (width 0.8) (layer B.Cu) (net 8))
 (segment (start 157.48 82.55) (end 160.02 82.55) (width 0.8) (layer B.Cu) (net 8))
 (segment (start 156.21 81.28) (end 157.48 82.55) (width 0.8) (layer B.Cu) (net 8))
 (segment (start 158.75 92.71) (end 158.75 102.87) (width 0.8) (layer B.Cu) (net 3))
 (segment (start 151.13 92.71) (end 151.13 102.87) (width 0.8) (layer B.Cu) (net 4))
 (segment (start 150.905 102.645) (end 151.13 102.87) (width 0.8) (layer B.Cu) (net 4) (status 30))
 (segment (start 142.55 146.05) (end 142.55 137.26) (width 0.8) (layer B.Cu) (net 14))
 (segment (start 142.55 137.26) (end 143.51 136.3) (width 0.8) (layer B.Cu) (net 14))
 (segment (start 143.185 136.625) (end 143.51 136.3) (width 0.8) (layer B.Cu) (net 14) (status 30)))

